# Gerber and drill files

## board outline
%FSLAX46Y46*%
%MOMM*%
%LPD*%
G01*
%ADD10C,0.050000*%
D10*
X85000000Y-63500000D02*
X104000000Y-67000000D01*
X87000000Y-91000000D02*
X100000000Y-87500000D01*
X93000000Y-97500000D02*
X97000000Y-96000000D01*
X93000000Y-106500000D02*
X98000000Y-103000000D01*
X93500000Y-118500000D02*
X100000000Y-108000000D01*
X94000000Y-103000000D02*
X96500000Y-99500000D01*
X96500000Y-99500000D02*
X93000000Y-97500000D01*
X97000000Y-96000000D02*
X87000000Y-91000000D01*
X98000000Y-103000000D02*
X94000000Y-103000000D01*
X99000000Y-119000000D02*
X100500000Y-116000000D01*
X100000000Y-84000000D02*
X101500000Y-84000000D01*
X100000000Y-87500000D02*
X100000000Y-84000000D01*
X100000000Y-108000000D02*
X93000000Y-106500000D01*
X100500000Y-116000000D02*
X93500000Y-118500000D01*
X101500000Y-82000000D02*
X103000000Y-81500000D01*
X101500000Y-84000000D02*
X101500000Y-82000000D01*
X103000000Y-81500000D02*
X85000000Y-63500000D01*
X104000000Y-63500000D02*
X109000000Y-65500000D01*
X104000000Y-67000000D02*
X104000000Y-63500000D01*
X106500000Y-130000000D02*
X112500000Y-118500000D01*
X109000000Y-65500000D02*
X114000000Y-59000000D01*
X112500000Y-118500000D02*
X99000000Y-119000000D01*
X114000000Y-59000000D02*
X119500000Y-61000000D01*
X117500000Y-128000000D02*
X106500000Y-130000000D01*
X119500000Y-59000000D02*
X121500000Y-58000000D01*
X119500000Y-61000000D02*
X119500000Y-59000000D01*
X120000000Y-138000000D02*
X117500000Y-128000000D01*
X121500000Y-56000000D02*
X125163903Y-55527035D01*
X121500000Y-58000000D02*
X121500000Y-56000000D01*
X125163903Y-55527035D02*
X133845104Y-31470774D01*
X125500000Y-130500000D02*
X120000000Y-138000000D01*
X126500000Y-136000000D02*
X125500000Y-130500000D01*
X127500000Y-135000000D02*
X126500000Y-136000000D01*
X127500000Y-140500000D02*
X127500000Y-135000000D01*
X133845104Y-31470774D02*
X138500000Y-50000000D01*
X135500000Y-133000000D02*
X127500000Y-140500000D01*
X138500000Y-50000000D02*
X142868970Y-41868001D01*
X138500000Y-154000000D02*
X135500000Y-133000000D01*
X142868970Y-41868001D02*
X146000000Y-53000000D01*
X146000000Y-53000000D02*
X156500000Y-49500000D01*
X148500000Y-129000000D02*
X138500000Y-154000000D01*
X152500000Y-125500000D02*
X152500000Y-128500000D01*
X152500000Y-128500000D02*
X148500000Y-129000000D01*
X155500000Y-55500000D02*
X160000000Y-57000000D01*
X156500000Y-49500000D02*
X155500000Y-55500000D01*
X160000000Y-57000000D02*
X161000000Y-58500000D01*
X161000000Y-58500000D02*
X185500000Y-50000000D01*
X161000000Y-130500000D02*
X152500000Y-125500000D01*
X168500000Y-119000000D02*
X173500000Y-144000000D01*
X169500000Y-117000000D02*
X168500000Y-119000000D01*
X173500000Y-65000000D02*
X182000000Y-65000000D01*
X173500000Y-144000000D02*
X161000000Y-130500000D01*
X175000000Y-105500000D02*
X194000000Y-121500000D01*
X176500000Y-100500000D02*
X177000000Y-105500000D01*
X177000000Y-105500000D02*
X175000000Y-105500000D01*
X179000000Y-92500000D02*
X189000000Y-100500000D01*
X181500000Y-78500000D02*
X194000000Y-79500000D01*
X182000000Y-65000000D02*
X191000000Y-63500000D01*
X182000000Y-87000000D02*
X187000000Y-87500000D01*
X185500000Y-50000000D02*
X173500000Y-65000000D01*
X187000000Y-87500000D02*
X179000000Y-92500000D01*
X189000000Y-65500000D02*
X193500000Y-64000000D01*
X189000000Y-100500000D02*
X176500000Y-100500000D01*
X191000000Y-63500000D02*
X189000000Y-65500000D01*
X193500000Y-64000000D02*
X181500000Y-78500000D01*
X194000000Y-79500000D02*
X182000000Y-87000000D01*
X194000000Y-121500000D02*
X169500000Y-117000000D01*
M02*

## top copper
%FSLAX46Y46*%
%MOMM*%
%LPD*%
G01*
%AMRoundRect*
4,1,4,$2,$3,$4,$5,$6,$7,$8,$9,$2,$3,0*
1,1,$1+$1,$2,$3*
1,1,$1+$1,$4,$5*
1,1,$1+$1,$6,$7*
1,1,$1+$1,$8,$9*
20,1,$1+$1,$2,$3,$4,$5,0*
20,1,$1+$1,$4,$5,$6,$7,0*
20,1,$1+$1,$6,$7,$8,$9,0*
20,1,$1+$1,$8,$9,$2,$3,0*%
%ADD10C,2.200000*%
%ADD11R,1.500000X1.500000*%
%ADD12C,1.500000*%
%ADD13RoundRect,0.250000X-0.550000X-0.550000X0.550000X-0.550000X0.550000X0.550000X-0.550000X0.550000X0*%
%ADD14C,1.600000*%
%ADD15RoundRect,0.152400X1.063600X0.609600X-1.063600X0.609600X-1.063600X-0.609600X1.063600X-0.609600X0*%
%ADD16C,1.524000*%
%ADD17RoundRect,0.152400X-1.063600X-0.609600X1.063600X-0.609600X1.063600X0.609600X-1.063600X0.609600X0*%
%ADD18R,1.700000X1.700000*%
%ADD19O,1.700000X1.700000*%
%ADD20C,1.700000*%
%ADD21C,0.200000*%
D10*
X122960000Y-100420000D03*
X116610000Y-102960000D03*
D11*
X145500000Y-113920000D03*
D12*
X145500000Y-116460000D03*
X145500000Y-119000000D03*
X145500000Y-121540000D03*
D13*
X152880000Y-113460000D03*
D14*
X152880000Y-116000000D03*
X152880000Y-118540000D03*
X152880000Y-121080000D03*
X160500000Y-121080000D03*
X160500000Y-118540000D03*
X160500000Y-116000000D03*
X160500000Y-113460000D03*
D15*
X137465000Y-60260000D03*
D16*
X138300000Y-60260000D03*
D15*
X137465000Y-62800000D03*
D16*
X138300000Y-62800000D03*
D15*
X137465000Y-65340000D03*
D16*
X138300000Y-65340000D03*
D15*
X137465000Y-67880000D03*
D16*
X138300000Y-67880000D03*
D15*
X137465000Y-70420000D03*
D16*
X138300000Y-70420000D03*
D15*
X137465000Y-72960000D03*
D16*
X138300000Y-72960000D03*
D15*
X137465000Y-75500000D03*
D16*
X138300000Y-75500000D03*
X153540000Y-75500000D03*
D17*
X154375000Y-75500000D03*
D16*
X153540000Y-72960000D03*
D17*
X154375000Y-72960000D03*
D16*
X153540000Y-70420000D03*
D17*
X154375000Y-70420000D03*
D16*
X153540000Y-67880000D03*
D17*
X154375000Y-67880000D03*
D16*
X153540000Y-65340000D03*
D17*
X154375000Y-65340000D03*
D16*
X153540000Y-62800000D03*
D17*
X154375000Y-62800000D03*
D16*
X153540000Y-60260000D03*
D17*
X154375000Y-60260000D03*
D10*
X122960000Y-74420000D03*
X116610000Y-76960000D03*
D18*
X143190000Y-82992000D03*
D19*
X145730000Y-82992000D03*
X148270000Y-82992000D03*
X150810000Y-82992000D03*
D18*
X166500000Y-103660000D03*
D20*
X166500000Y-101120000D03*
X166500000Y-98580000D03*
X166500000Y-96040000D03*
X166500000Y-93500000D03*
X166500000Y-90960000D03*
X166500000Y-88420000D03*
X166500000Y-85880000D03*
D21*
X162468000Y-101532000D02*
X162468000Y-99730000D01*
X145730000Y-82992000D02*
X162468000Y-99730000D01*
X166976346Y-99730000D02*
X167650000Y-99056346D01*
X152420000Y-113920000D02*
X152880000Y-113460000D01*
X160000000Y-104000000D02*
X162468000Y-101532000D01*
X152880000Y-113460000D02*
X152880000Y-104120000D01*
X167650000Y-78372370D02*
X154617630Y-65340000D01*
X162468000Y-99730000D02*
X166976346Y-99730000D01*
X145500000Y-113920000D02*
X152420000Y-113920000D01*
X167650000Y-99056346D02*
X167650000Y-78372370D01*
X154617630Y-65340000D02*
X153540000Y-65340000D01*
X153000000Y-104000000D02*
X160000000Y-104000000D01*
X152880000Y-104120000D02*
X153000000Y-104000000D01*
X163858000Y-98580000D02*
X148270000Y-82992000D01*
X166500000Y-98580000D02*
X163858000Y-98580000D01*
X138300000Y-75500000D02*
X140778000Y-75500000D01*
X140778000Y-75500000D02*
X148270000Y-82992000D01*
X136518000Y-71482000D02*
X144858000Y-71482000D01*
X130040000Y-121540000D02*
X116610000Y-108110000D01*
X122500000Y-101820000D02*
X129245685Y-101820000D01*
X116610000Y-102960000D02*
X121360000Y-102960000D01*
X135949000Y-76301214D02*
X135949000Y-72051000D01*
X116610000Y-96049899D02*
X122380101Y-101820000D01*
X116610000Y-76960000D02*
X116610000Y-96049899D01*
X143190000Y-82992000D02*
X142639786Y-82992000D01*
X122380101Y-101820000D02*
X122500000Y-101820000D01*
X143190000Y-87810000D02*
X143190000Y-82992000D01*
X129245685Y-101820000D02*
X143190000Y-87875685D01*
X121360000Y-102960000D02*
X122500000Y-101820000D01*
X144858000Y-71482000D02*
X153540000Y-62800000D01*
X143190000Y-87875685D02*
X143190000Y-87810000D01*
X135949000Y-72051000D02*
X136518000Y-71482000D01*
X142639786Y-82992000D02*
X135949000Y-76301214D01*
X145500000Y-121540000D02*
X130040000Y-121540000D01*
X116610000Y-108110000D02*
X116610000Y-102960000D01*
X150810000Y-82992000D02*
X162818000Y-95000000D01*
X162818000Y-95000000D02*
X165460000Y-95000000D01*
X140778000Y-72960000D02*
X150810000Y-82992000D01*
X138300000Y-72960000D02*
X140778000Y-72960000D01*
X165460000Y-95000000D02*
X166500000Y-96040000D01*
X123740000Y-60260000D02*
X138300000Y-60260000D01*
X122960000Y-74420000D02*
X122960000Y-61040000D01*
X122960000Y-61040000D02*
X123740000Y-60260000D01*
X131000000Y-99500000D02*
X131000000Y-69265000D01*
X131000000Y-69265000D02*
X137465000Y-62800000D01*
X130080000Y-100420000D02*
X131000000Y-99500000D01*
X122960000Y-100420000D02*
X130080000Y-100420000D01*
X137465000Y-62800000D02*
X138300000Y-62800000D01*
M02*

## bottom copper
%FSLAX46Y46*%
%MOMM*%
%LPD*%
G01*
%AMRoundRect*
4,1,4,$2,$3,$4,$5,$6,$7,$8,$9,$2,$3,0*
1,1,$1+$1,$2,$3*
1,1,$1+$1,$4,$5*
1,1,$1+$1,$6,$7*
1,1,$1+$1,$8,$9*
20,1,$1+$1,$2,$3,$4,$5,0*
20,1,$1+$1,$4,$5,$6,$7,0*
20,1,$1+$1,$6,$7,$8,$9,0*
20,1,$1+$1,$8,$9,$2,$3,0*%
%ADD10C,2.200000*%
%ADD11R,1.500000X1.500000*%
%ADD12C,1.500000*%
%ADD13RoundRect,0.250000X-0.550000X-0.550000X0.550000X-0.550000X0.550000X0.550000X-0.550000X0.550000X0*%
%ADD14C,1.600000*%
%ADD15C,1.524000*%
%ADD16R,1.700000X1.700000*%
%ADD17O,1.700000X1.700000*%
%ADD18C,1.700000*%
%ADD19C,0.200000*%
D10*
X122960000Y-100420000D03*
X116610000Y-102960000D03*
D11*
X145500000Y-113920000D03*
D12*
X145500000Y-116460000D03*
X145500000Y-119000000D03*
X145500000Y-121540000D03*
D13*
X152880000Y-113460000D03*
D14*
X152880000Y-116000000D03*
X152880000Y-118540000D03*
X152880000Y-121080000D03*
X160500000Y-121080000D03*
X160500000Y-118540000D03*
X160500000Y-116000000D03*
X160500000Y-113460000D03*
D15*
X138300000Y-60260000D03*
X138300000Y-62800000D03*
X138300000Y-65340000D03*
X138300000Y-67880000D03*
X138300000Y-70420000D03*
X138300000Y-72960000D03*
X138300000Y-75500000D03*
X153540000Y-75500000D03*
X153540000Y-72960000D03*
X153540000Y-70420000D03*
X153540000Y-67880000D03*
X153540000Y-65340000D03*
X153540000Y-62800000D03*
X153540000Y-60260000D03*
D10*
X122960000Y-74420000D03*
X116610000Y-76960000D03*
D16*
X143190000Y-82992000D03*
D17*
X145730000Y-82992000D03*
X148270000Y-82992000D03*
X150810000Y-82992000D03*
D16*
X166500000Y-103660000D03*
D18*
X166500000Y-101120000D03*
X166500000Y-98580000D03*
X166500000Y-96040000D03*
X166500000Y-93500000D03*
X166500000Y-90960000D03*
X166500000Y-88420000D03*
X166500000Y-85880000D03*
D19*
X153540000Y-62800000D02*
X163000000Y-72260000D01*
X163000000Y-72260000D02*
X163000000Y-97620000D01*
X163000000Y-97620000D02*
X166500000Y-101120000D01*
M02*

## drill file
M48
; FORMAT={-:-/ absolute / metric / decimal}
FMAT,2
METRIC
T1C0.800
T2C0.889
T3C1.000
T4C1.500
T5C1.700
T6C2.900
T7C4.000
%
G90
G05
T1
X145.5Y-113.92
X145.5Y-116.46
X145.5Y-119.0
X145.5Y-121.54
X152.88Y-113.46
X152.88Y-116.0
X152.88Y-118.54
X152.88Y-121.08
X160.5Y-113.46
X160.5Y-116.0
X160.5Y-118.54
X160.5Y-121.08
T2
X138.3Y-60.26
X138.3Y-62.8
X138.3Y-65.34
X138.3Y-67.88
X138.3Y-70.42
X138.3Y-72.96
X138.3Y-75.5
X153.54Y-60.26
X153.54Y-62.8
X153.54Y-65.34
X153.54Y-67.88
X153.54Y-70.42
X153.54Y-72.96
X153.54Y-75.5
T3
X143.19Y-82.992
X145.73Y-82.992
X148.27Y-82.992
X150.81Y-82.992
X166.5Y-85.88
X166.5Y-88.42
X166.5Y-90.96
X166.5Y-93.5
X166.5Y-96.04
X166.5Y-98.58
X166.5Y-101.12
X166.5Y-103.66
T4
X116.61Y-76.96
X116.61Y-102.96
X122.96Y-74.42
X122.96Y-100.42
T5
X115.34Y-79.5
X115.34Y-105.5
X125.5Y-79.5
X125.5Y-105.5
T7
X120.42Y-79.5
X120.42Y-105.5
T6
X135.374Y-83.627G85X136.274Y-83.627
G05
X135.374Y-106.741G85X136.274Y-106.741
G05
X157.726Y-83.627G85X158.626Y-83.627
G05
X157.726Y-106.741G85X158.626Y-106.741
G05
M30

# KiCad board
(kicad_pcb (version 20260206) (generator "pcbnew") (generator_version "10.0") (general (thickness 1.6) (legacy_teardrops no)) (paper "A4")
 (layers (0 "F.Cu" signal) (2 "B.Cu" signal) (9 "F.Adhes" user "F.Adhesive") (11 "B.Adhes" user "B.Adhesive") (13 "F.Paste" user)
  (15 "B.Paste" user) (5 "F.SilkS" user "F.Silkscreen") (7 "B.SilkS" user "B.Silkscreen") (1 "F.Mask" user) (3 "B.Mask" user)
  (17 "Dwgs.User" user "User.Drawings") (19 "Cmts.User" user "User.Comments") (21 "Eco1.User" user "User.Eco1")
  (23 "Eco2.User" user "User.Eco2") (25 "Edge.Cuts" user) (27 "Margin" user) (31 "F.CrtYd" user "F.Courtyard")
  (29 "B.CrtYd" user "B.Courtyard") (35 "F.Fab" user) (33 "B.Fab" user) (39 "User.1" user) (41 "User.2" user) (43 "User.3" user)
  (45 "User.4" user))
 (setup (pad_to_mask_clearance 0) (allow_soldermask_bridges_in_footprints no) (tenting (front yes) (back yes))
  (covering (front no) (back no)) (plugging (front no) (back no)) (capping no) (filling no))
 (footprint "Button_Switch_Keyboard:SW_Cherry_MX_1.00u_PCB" (layer "F.Cu") (at 122.96 100.42)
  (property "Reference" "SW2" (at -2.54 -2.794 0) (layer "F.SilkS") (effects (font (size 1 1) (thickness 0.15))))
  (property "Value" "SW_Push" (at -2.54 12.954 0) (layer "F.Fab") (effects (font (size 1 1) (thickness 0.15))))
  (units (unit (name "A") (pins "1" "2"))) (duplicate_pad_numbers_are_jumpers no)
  (pad "" np_thru_hole circle (at -7.62 5.08) (size 1.7 1.7) (drill 1.7) (layers "*.Cu" "*.Mask"))
  (pad "" np_thru_hole circle (at -2.54 5.08) (size 4 4) (drill 4) (layers "*.Cu" "*.Mask"))
  (pad "" np_thru_hole circle (at 2.54 5.08) (size 1.7 1.7) (drill 1.7) (layers "*.Cu" "*.Mask"))
  (pad "1" thru_hole circle (at 0 0) (size 2.2 2.2) (drill 1.5) (layers "*.Cu" "*.Mask") (remove_unused_layers no) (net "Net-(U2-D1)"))
  (pad "2" thru_hole circle (at -6.35 2.54) (size 2.2 2.2) (drill 1.5) (layers "*.Cu" "*.Mask") (remove_unused_layers no) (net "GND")))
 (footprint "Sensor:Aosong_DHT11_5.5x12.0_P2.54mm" (layer "F.Cu") (at 145.5 113.92)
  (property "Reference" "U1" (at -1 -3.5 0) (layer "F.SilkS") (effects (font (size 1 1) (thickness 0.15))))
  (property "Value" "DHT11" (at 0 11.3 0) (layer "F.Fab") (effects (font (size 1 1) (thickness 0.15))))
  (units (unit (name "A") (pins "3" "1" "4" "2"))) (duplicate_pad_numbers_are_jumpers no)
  (pad "1" thru_hole rect (at 0 0) (size 1.5 1.5) (drill 0.8) (layers "*.Cu" "*.Mask") (remove_unused_layers no) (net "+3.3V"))
  (pad "2" thru_hole circle (at 0 2.54) (size 1.5 1.5) (drill 0.8) (layers "*.Cu" "*.Mask") (remove_unused_layers no)
   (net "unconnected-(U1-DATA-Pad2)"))
  (pad "3" thru_hole circle (at 0 5.08) (size 1.5 1.5) (drill 0.8) (layers "*.Cu" "*.Mask") (remove_unused_layers no)
   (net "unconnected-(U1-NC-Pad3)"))
  (pad "4" thru_hole circle (at 0 7.62) (size 1.5 1.5) (drill 0.8) (layers "*.Cu" "*.Mask") (remove_unused_layers no) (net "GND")))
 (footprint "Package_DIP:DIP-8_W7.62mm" (layer "F.Cu") (at 152.88 113.46)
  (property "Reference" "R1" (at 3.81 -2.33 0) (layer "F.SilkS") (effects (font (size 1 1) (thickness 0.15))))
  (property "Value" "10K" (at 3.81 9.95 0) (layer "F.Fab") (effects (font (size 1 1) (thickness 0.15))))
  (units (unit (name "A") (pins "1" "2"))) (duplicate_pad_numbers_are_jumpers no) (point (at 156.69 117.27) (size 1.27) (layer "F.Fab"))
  (pad "1" thru_hole roundrect (at 0 0) (size 1.6 1.6) (drill 0.8) (layers "*.Cu" "*.Mask") (remove_unused_layers no)
   (roundrect_rratio 0.15625) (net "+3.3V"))
  (pad "2" thru_hole circle (at 0 2.54) (size 1.6 1.6) (drill 0.8) (layers "*.Cu" "*.Mask") (remove_unused_layers no) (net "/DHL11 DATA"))
  (pad "3" thru_hole circle (at 0 5.08) (size 1.6 1.6) (drill 0.8) (layers "*.Cu" "*.Mask") (remove_unused_layers no))
  (pad "4" thru_hole circle (at 0 7.62) (size 1.6 1.6) (drill 0.8) (layers "*.Cu" "*.Mask") (remove_unused_layers no))
  (pad "5" thru_hole circle (at 7.62 7.62) (size 1.6 1.6) (drill 0.8) (layers "*.Cu" "*.Mask") (remove_unused_layers no))
  (pad "6" thru_hole circle (at 7.62 5.08) (size 1.6 1.6) (drill 0.8) (layers "*.Cu" "*.Mask") (remove_unused_layers no))
  (pad "7" thru_hole circle (at 7.62 2.54) (size 1.6 1.6) (drill 0.8) (layers "*.Cu" "*.Mask") (remove_unused_layers no))
  (pad "8" thru_hole circle (at 7.62 0) (size 1.6 1.6) (drill 0.8) (layers "*.Cu" "*.Mask") (remove_unused_layers no)))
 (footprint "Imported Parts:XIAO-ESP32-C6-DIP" (layer "F.Cu") (at 145.92 67.88 90)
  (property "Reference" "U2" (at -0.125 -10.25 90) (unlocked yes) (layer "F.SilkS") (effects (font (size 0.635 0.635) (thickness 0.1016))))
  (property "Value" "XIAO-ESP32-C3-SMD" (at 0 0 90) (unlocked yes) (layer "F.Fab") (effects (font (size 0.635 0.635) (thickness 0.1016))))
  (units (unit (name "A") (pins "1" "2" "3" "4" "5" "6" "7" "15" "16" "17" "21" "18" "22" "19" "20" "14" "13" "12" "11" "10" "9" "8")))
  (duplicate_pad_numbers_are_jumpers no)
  (pad "1" smd roundrect (at 7.62 -8.455 180) (size 2.432 1.524) (layers "F.Cu" "F.Mask") (roundrect_rratio 0.1) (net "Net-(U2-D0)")
   (thermal_bridge_angle 45))
  (pad "1" thru_hole circle (at 7.62 -7.62 180) (size 1.524 1.524) (drill 0.889) (layers "*.Cu" "*.Mask") (remove_unused_layers no)
   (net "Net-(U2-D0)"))
  (pad "2" smd roundrect (at 5.08 -8.455 180) (size 2.432 1.524) (layers "F.Cu" "F.Mask") (roundrect_rratio 0.1) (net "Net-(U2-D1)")
   (thermal_bridge_angle 45))
  (pad "2" thru_hole circle (at 5.08 -7.62 180) (size 1.524 1.524) (drill 0.889) (layers "*.Cu" "*.Mask") (remove_unused_layers no)
   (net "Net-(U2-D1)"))
  (pad "3" smd roundrect (at 2.54 -8.455 180) (size 2.432 1.524) (layers "F.Cu" "F.Mask") (roundrect_rratio 0.1)
   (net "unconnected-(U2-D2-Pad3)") (thermal_bridge_angle 45))
  (pad "3" thru_hole circle (at 2.54 -7.62 180) (size 1.524 1.524) (drill 0.889) (layers "*.Cu" "*.Mask") (remove_unused_layers no)
   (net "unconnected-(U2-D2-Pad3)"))
  (pad "4" smd roundrect (at 0 -8.455 180) (size 2.432 1.524) (layers "F.Cu" "F.Mask") (roundrect_rratio 0.1)
   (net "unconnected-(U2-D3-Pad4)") (thermal_bridge_angle 45))
  (pad "4" thru_hole circle (at 0 -7.62 180) (size 1.524 1.524) (drill 0.889) (layers "*.Cu" "*.Mask") (remove_unused_layers no)
   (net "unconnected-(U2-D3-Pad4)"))
  (pad "5" smd roundrect (at -2.54 -8.455 180) (size 2.432 1.524) (layers "F.Cu" "F.Mask") (roundrect_rratio 0.1)
   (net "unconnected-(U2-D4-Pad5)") (thermal_bridge_angle 45))
  (pad "5" thru_hole circle (at -2.54 -7.62 180) (size 1.524 1.524) (drill 0.889) (layers "*.Cu" "*.Mask") (remove_unused_layers no)
   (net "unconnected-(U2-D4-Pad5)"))
  (pad "6" smd roundrect (at -5.08 -8.455 180) (size 2.432 1.524) (layers "F.Cu" "F.Mask") (roundrect_rratio 0.1) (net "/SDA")
   (thermal_bridge_angle 45))
  (pad "6" thru_hole circle (at -5.08 -7.62 180) (size 1.524 1.524) (drill 0.889) (layers "*.Cu" "*.Mask") (remove_unused_layers no)
   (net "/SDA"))
  (pad "7" smd roundrect (at -7.62 -8.455 180) (size 2.432 1.524) (layers "F.Cu" "F.Mask") (roundrect_rratio 0.1) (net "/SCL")
   (thermal_bridge_angle 45))
  (pad "7" thru_hole circle (at -7.62 -7.62 180) (size 1.524 1.524) (drill 0.889) (layers "*.Cu" "*.Mask") (remove_unused_layers no)
   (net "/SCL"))
  (pad "8" thru_hole circle (at -7.62 7.62) (size 1.524 1.524) (drill 0.889) (layers "*.Cu" "*.Mask") (remove_unused_layers no)
   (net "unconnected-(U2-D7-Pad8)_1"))
  (pad "8" smd roundrect (at -7.62 8.455) (size 2.432 1.524) (layers "F.Cu" "F.Mask") (roundrect_rratio 0.1)
   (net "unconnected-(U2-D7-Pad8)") (thermal_bridge_angle 45))
  (pad "9" thru_hole circle (at -5.08 7.62) (size 1.524 1.524) (drill 0.889) (layers "*.Cu" "*.Mask") (remove_unused_layers no)
   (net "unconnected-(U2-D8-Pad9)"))
  (pad "9" smd roundrect (at -5.08 8.455) (size 2.432 1.524) (layers "F.Cu" "F.Mask") (roundrect_rratio 0.1)
   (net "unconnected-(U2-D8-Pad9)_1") (thermal_bridge_angle 45))
  (pad "10" thru_hole circle (at -2.54 7.62) (size 1.524 1.524) (drill 0.889) (layers "*.Cu" "*.Mask") (remove_unused_layers no)
   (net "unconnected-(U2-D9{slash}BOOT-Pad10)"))
  (pad "10" smd roundrect (at -2.54 8.455) (size 2.432 1.524) (layers "F.Cu" "F.Mask") (roundrect_rratio 0.1)
   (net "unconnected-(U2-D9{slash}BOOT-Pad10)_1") (thermal_bridge_angle 45))
  (pad "11" thru_hole circle (at 0 7.62) (size 1.524 1.524) (drill 0.889) (layers "*.Cu" "*.Mask") (remove_unused_layers no)
   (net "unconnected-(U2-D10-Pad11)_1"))
  (pad "11" smd roundrect (at 0 8.455) (size 2.432 1.524) (layers "F.Cu" "F.Mask") (roundrect_rratio 0.1) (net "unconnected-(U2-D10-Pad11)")
   (thermal_bridge_angle 45))
  (pad "12" thru_hole circle (at 2.54 7.62) (size 1.524 1.524) (drill 0.889) (layers "*.Cu" "*.Mask") (remove_unused_layers no)
   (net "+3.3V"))
  (pad "12" smd roundrect (at 2.54 8.455) (size 2.432 1.524) (layers "F.Cu" "F.Mask") (roundrect_rratio 0.1) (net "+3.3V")
   (thermal_bridge_angle 45))
  (pad "13" thru_hole circle (at 5.08 7.62) (size 1.524 1.524) (drill 0.889) (layers "*.Cu" "*.Mask") (remove_unused_layers no) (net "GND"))
  (pad "13" smd roundrect (at 5.08 8.455) (size 2.432 1.524) (layers "F.Cu" "F.Mask") (roundrect_rratio 0.1) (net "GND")
   (thermal_bridge_angle 45))
  (pad "14" thru_hole circle (at 7.62 7.62) (size 1.524 1.524) (drill 0.889) (layers "*.Cu" "*.Mask") (remove_unused_layers no) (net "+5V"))
  (pad "14" smd roundrect (at 7.62 8.455) (size 2.432 1.524) (layers "F.Cu" "F.Mask") (roundrect_rratio 0.1) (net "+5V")
   (thermal_bridge_angle 45)))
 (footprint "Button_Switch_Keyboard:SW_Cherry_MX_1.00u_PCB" (layer "F.Cu") (at 122.96 74.42)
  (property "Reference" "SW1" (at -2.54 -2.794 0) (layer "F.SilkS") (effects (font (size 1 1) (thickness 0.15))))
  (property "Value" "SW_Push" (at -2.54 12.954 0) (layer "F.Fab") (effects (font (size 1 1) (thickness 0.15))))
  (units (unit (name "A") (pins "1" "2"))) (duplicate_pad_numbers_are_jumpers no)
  (pad "" np_thru_hole circle (at -7.62 5.08) (size 1.7 1.7) (drill 1.7) (layers "*.Cu" "*.Mask"))
  (pad "" np_thru_hole circle (at -2.54 5.08) (size 4 4) (drill 4) (layers "*.Cu" "*.Mask"))
  (pad "" np_thru_hole circle (at 2.54 5.08) (size 1.7 1.7) (drill 1.7) (layers "*.Cu" "*.Mask"))
  (pad "1" thru_hole circle (at 0 0) (size 2.2 2.2) (drill 1.5) (layers "*.Cu" "*.Mask") (remove_unused_layers no) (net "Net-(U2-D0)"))
  (pad "2" thru_hole circle (at -6.35 2.54) (size 2.2 2.2) (drill 1.5) (layers "*.Cu" "*.Mask") (remove_unused_layers no) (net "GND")))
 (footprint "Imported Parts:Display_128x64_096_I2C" (layer "F.Cu") (at 147 82.992)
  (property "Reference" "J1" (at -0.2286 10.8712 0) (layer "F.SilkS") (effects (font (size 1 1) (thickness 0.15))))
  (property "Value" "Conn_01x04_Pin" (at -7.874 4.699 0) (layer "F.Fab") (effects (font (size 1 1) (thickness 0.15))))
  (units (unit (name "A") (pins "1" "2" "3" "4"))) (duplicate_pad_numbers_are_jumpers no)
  (pad "" np_thru_hole oval (at -11.176 0.635) (size 3.8 2.9) (drill oval 3.8 2.9) (layers "*.Cu" "*.Mask"))
  (pad "" np_thru_hole oval (at -11.176 23.749) (size 3.8 2.9) (drill oval 3.8 2.9) (layers "*.Cu" "*.Mask"))
  (pad "" np_thru_hole oval (at 11.176 0.635) (size 3.8 2.9) (drill oval 3.8 2.9) (layers "*.Cu" "*.Mask"))
  (pad "" np_thru_hole oval (at 11.176 23.749) (size 3.8 2.9) (drill oval 3.8 2.9) (layers "*.Cu" "*.Mask"))
  (pad "1" thru_hole rect (at -3.81 0 90) (size 1.7 1.7) (drill 1) (layers "*.Cu" "*.Mask") (remove_unused_layers no) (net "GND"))
  (pad "2" thru_hole oval (at -1.27 0 90) (size 1.7 1.7) (drill 1) (layers "*.Cu" "*.Mask") (remove_unused_layers no) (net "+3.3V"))
  (pad "3" thru_hole oval (at 1.27 0 90) (size 1.7 1.7) (drill 1) (layers "*.Cu" "*.Mask") (remove_unused_layers no) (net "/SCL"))
  (pad "4" thru_hole oval (at 3.81 0 90) (size 1.7 1.7) (drill 1) (layers "*.Cu" "*.Mask") (remove_unused_layers no) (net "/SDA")))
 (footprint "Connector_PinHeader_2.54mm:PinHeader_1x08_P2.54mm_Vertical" (layer "F.Cu") (at 166.5 103.66 180)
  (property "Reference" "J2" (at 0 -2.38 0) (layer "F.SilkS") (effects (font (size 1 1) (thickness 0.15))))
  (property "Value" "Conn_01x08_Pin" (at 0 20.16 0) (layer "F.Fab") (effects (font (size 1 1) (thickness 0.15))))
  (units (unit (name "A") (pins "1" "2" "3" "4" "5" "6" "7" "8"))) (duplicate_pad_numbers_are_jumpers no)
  (pad "1" thru_hole rect (at 0 0 180) (size 1.7 1.7) (drill 1) (layers "*.Cu" "*.Mask") (remove_unused_layers no) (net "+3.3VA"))
  (pad "2" thru_hole circle (at 0 2.54 180) (size 1.7 1.7) (drill 1) (layers "*.Cu" "*.Mask") (remove_unused_layers no) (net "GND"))
  (pad "3" thru_hole circle (at 0 5.08 180) (size 1.7 1.7) (drill 1) (layers "*.Cu" "*.Mask") (remove_unused_layers no) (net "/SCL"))
  (pad "4" thru_hole circle (at 0 7.62 180) (size 1.7 1.7) (drill 1) (layers "*.Cu" "*.Mask") (remove_unused_layers no) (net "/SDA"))
  (pad "5" thru_hole circle (at 0 10.16 180) (size 1.7 1.7) (drill 1) (layers "*.Cu" "*.Mask") (remove_unused_layers no)
   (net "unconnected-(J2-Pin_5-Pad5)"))
  (pad "6" thru_hole circle (at 0 12.7 180) (size 1.7 1.7) (drill 1) (layers "*.Cu" "*.Mask") (remove_unused_layers no)
   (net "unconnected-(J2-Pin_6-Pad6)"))
  (pad "7" thru_hole circle (at 0 15.24 180) (size 1.7 1.7) (drill 1) (layers "*.Cu" "*.Mask") (remove_unused_layers no)
   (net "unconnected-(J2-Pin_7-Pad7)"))
  (pad "8" thru_hole circle (at 0 17.78 180) (size 1.7 1.7) (drill 1) (layers "*.Cu" "*.Mask") (remove_unused_layers no)
   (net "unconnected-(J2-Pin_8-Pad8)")))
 (gr_line (start 85 63.5) (end 104 67) (stroke (width 0.05) (type default)) (layer "Edge.Cuts"))
 (gr_line (start 87 91) (end 100 87.5) (stroke (width 0.05) (type default)) (layer "Edge.Cuts"))
 (gr_line (start 93 97.5) (end 97 96) (stroke (width 0.05) (type default)) (layer "Edge.Cuts"))
 (gr_line (start 93 106.5) (end 98 103) (stroke (width 0.05) (type default)) (layer "Edge.Cuts"))
 (gr_line (start 93.5 118.5) (end 100 108) (stroke (width 0.05) (type default)) (layer "Edge.Cuts"))
 (gr_line (start 94 103) (end 96.5 99.5) (stroke (width 0.05) (type default)) (layer "Edge.Cuts"))
 (gr_line (start 96.5 99.5) (end 93 97.5) (stroke (width 0.05) (type default)) (layer "Edge.Cuts"))
 (gr_line (start 97 96) (end 87 91) (stroke (width 0.05) (type default)) (layer "Edge.Cuts"))
 (gr_line (start 98 103) (end 94 103) (stroke (width 0.05) (type default)) (layer "Edge.Cuts"))
 (gr_line (start 99 119) (end 100.5 116) (stroke (width 0.05) (type default)) (layer "Edge.Cuts"))
 (gr_line (start 100 84) (end 101.5 84) (stroke (width 0.05) (type default)) (layer "Edge.Cuts"))
 (gr_line (start 100 87.5) (end 100 84) (stroke (width 0.05) (type default)) (layer "Edge.Cuts"))
 (gr_line (start 100 108) (end 93 106.5) (stroke (width 0.05) (type default)) (layer "Edge.Cuts"))
 (gr_line (start 100.5 116) (end 93.5 118.5) (stroke (width 0.05) (type default)) (layer "Edge.Cuts"))
 (gr_line (start 101.5 82) (end 103 81.5) (stroke (width 0.05) (type default)) (layer "Edge.Cuts"))
 (gr_line (start 101.5 84) (end 101.5 82) (stroke (width 0.05) (type default)) (layer "Edge.Cuts"))
 (gr_line (start 103 81.5) (end 85 63.5) (stroke (width 0.05) (type default)) (layer "Edge.Cuts"))
 (gr_line (start 104 63.5) (end 109 65.5) (stroke (width 0.05) (type default)) (layer "Edge.Cuts"))
 (gr_line (start 104 67) (end 104 63.5) (stroke (width 0.05) (type default)) (layer "Edge.Cuts"))
 (gr_line (start 106.5 130) (end 112.5 118.5) (stroke (width 0.05) (type default)) (layer "Edge.Cuts"))
 (gr_line (start 109 65.5) (end 114 59) (stroke (width 0.05) (type default)) (layer "Edge.Cuts"))
 (gr_line (start 112.5 118.5) (end 99 119) (stroke (width 0.05) (type default)) (layer "Edge.Cuts"))
 (gr_line (start 114 59) (end 119.5 61) (stroke (width 0.05) (type default)) (layer "Edge.Cuts"))
 (gr_line (start 117.5 128) (end 106.5 130) (stroke (width 0.05) (type default)) (layer "Edge.Cuts"))
 (gr_line (start 119.5 59) (end 121.5 58) (stroke (width 0.05) (type default)) (layer "Edge.Cuts"))
 (gr_line (start 119.5 61) (end 119.5 59) (stroke (width 0.05) (type default)) (layer "Edge.Cuts"))
 (gr_line (start 120 138) (end 117.5 128) (stroke (width 0.05) (type default)) (layer "Edge.Cuts"))
 (gr_line (start 121.5 56) (end 125.163903 55.527035) (stroke (width 0.05) (type default)) (layer "Edge.Cuts"))
 (gr_line (start 121.5 58) (end 121.5 56) (stroke (width 0.05) (type default)) (layer "Edge.Cuts"))
 (gr_line (start 125.163903 55.527035) (end 133.845104 31.470774) (stroke (width 0.05) (type default)) (layer "Edge.Cuts"))
 (gr_line (start 125.5 130.5) (end 120 138) (stroke (width 0.05) (type default)) (layer "Edge.Cuts"))
 (gr_line (start 126.5 136) (end 125.5 130.5) (stroke (width 0.05) (type default)) (layer "Edge.Cuts"))
 (gr_line (start 127.5 135) (end 126.5 136) (stroke (width 0.05) (type default)) (layer "Edge.Cuts"))
 (gr_line (start 127.5 140.5) (end 127.5 135) (stroke (width 0.05) (type default)) (layer "Edge.Cuts"))
 (gr_line (start 133.845104 31.470774) (end 138.5 50) (stroke (width 0.05) (type default)) (layer "Edge.Cuts"))
 (gr_line (start 135.5 133) (end 127.5 140.5) (stroke (width 0.05) (type default)) (layer "Edge.Cuts"))
 (gr_line (start 138.5 50) (end 142.86897 41.868001) (stroke (width 0.05) (type default)) (layer "Edge.Cuts"))
 (gr_line (start 138.5 154) (end 135.5 133) (stroke (width 0.05) (type default)) (layer "Edge.Cuts"))
 (gr_line (start 142.86897 41.868001) (end 146 53) (stroke (width 0.05) (type default)) (layer "Edge.Cuts"))
 (gr_line (start 146 53) (end 156.5 49.5) (stroke (width 0.05) (type default)) (layer "Edge.Cuts"))
 (gr_line (start 148.5 129) (end 138.5 154) (stroke (width 0.05) (type default)) (layer "Edge.Cuts"))
 (gr_line (start 152.5 125.5) (end 152.5 128.5) (stroke (width 0.05) (type default)) (layer "Edge.Cuts"))
 (gr_line (start 152.5 128.5) (end 148.5 129) (stroke (width 0.05) (type default)) (layer "Edge.Cuts"))
 (gr_line (start 155.5 55.5) (end 160 57) (stroke (width 0.05) (type default)) (layer "Edge.Cuts"))
 (gr_line (start 156.5 49.5) (end 155.5 55.5) (stroke (width 0.05) (type default)) (layer "Edge.Cuts"))
 (gr_line (start 160 57) (end 161 58.5) (stroke (width 0.05) (type default)) (layer "Edge.Cuts"))
 (gr_line (start 161 58.5) (end 185.5 50) (stroke (width 0.05) (type default)) (layer "Edge.Cuts"))
 (gr_line (start 161 130.5) (end 152.5 125.5) (stroke (width 0.05) (type default)) (layer "Edge.Cuts"))
 (gr_line (start 168.5 119) (end 173.5 144) (stroke (width 0.05) (type default)) (layer "Edge.Cuts"))
 (gr_line (start 169.5 117) (end 168.5 119) (stroke (width 0.05) (type default)) (layer "Edge.Cuts"))
 (gr_line (start 173.5 65) (end 182 65) (stroke (width 0.05) (type default)) (layer "Edge.Cuts"))
 (gr_line (start 173.5 144) (end 161 130.5) (stroke (width 0.05) (type default)) (layer "Edge.Cuts"))
 (gr_line (start 175 105.5) (end 194 121.5) (stroke (width 0.05) (type default)) (layer "Edge.Cuts"))
 (gr_line (start 176.5 100.5) (end 177 105.5) (stroke (width 0.05) (type default)) (layer "Edge.Cuts"))
 (gr_line (start 177 105.5) (end 175 105.5) (stroke (width 0.05) (type default)) (layer "Edge.Cuts"))
 (gr_line (start 179 92.5) (end 189 100.5) (stroke (width 0.05) (type default)) (layer "Edge.Cuts"))
 (gr_line (start 181.5 78.5) (end 194 79.5) (stroke (width 0.05) (type default)) (layer "Edge.Cuts"))
 (gr_line (start 182 65) (end 191 63.5) (stroke (width 0.05) (type default)) (layer "Edge.Cuts"))
 (gr_line (start 182 87) (end 187 87.5) (stroke (width 0.05) (type default)) (layer "Edge.Cuts"))
 (gr_line (start 185.5 50) (end 173.5 65) (stroke (width 0.05) (type default)) (layer "Edge.Cuts"))
 (gr_line (start 187 87.5) (end 179 92.5) (stroke (width 0.05) (type default)) (layer "Edge.Cuts"))
 (gr_line (start 189 65.5) (end 193.5 64) (stroke (width 0.05) (type default)) (layer "Edge.Cuts"))
 (gr_line (start 189 100.5) (end 176.5 100.5) (stroke (width 0.05) (type default)) (layer "Edge.Cuts"))
 (gr_line (start 191 63.5) (end 189 65.5) (stroke (width 0.05) (type default)) (layer "Edge.Cuts"))
 (gr_line (start 193.5 64) (end 181.5 78.5) (stroke (width 0.05) (type default)) (layer "Edge.Cuts"))
 (gr_line (start 194 79.5) (end 182 87) (stroke (width 0.05) (type default)) (layer "Edge.Cuts"))
 (gr_line (start 194 121.5) (end 169.5 117) (stroke (width 0.05) (type default)) (layer "Edge.Cuts"))
 (segment (start 162.468 101.532) (end 162.468 99.73) (width 0.2) (layer "F.Cu") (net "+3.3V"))
 (segment (start 145.73 82.992) (end 162.468 99.73) (width 0.2) (layer "F.Cu") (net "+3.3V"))
 (segment (start 166.976346 99.73) (end 167.65 99.056346) (width 0.2) (layer "F.Cu") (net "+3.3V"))
 (segment (start 152.42 113.92) (end 152.88 113.46) (width 0.2) (layer "F.Cu") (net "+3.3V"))
 (segment (start 160 104) (end 162.468 101.532) (width 0.2) (layer "F.Cu") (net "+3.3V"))
 (segment (start 152.88 113.46) (end 152.88 104.12) (width 0.2) (layer "F.Cu") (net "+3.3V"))
 (segment (start 167.65 78.37237) (end 154.61763 65.34) (width 0.2) (layer "F.Cu") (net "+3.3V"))
 (segment (start 162.468 99.73) (end 166.976346 99.73) (width 0.2) (layer "F.Cu") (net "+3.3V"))
 (segment (start 145.5 113.92) (end 152.42 113.92) (width 0.2) (layer "F.Cu") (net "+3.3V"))
 (segment (start 167.65 99.056346) (end 167.65 78.37237) (width 0.2) (layer "F.Cu") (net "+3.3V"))
 (segment (start 154.61763 65.34) (end 153.54 65.34) (width 0.2) (layer "F.Cu") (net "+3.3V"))
 (segment (start 153 104) (end 160 104) (width 0.2) (layer "F.Cu") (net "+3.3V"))
 (segment (start 152.88 104.12) (end 153 104) (width 0.2) (layer "F.Cu") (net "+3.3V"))
 (segment (start 163.858 98.58) (end 148.27 82.992) (width 0.2) (layer "F.Cu") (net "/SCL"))
 (segment (start 166.5 98.58) (end 163.858 98.58) (width 0.2) (layer "F.Cu") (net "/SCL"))
 (segment (start 138.3 75.5) (end 140.778 75.5) (width 0.2) (layer "F.Cu") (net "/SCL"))
 (segment (start 140.778 75.5) (end 148.27 82.992) (width 0.2) (layer "F.Cu") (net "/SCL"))
 (segment (start 136.518 71.482) (end 144.858 71.482) (width 0.2) (layer "F.Cu") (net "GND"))
 (segment (start 130.04 121.54) (end 116.61 108.11) (width 0.2) (layer "F.Cu") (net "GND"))
 (segment (start 122.5 101.82) (end 129.245685 101.82) (width 0.2) (layer "F.Cu") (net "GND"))
 (segment (start 116.61 102.96) (end 121.36 102.96) (width 0.2) (layer "F.Cu") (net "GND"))
 (segment (start 135.949 76.301214) (end 135.949 72.051) (width 0.2) (layer "F.Cu") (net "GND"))
 (segment (start 116.61 96.049899) (end 122.380101 101.82) (width 0.2) (layer "F.Cu") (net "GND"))
 (segment (start 116.61 76.96) (end 116.61 96.049899) (width 0.2) (layer "F.Cu") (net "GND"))
 (segment (start 143.19 82.992) (end 142.639786 82.992) (width 0.2) (layer "F.Cu") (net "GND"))
 (segment (start 122.380101 101.82) (end 122.5 101.82) (width 0.2) (layer "F.Cu") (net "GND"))
 (segment (start 143.19 87.81) (end 143.19 82.992) (width 0.2) (layer "F.Cu") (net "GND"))
 (segment (start 129.245685 101.82) (end 143.19 87.875685) (width 0.2) (layer "F.Cu") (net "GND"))
 (segment (start 121.36 102.96) (end 122.5 101.82) (width 0.2) (layer "F.Cu") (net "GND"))
 (segment (start 144.858 71.482) (end 153.54 62.8) (width 0.2) (layer "F.Cu") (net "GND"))
 (segment (start 143.19 87.875685) (end 143.19 87.81) (width 0.2) (layer "F.Cu") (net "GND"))
 (segment (start 135.949 72.051) (end 136.518 71.482) (width 0.2) (layer "F.Cu") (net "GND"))
 (segment (start 142.639786 82.992) (end 135.949 76.301214) (width 0.2) (layer "F.Cu") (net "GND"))
 (segment (start 145.5 121.54) (end 130.04 121.54) (width 0.2) (layer "F.Cu") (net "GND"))
 (segment (start 116.61 108.11) (end 116.61 102.96) (width 0.2) (layer "F.Cu") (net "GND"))
 (segment (start 153.54 62.8) (end 163 72.26) (width 0.2) (layer "B.Cu") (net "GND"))
 (segment (start 163 72.26) (end 163 97.62) (width 0.2) (layer "B.Cu") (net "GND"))
 (segment (start 163 97.62) (end 166.5 101.12) (width 0.2) (layer "B.Cu") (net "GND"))
 (segment (start 150.81 82.992) (end 162.818 95) (width 0.2) (layer "F.Cu") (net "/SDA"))
 (segment (start 162.818 95) (end 165.46 95) (width 0.2) (layer "F.Cu") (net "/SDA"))
 (segment (start 140.778 72.96) (end 150.81 82.992) (width 0.2) (layer "F.Cu") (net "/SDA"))
 (segment (start 138.3 72.96) (end 140.778 72.96) (width 0.2) (layer "F.Cu") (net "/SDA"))
 (segment (start 165.46 95) (end 166.5 96.04) (width 0.2) (layer "F.Cu") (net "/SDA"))
 (segment (start 123.74 60.26) (end 138.3 60.26) (width 0.2) (layer "F.Cu") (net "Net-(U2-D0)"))
 (segment (start 122.96 74.42) (end 122.96 61.04) (width 0.2) (layer "F.Cu") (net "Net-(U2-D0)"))
 (segment (start 122.96 61.04) (end 123.74 60.26) (width 0.2) (layer "F.Cu") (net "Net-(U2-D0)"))
 (segment (start 131 99.5) (end 131 69.265) (width 0.2) (layer "F.Cu") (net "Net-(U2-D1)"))
 (segment (start 131 69.265) (end 137.465 62.8) (width 0.2) (layer "F.Cu") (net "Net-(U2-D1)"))
 (segment (start 130.08 100.42) (end 131 99.5) (width 0.2) (layer "F.Cu") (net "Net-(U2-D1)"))
 (segment (start 122.96 100.42) (end 130.08 100.42) (width 0.2) (layer "F.Cu") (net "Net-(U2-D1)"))
 (segment (start 137.465 62.8) (end 138.3 62.8) (width 0.2) (layer "F.Cu") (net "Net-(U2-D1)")))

